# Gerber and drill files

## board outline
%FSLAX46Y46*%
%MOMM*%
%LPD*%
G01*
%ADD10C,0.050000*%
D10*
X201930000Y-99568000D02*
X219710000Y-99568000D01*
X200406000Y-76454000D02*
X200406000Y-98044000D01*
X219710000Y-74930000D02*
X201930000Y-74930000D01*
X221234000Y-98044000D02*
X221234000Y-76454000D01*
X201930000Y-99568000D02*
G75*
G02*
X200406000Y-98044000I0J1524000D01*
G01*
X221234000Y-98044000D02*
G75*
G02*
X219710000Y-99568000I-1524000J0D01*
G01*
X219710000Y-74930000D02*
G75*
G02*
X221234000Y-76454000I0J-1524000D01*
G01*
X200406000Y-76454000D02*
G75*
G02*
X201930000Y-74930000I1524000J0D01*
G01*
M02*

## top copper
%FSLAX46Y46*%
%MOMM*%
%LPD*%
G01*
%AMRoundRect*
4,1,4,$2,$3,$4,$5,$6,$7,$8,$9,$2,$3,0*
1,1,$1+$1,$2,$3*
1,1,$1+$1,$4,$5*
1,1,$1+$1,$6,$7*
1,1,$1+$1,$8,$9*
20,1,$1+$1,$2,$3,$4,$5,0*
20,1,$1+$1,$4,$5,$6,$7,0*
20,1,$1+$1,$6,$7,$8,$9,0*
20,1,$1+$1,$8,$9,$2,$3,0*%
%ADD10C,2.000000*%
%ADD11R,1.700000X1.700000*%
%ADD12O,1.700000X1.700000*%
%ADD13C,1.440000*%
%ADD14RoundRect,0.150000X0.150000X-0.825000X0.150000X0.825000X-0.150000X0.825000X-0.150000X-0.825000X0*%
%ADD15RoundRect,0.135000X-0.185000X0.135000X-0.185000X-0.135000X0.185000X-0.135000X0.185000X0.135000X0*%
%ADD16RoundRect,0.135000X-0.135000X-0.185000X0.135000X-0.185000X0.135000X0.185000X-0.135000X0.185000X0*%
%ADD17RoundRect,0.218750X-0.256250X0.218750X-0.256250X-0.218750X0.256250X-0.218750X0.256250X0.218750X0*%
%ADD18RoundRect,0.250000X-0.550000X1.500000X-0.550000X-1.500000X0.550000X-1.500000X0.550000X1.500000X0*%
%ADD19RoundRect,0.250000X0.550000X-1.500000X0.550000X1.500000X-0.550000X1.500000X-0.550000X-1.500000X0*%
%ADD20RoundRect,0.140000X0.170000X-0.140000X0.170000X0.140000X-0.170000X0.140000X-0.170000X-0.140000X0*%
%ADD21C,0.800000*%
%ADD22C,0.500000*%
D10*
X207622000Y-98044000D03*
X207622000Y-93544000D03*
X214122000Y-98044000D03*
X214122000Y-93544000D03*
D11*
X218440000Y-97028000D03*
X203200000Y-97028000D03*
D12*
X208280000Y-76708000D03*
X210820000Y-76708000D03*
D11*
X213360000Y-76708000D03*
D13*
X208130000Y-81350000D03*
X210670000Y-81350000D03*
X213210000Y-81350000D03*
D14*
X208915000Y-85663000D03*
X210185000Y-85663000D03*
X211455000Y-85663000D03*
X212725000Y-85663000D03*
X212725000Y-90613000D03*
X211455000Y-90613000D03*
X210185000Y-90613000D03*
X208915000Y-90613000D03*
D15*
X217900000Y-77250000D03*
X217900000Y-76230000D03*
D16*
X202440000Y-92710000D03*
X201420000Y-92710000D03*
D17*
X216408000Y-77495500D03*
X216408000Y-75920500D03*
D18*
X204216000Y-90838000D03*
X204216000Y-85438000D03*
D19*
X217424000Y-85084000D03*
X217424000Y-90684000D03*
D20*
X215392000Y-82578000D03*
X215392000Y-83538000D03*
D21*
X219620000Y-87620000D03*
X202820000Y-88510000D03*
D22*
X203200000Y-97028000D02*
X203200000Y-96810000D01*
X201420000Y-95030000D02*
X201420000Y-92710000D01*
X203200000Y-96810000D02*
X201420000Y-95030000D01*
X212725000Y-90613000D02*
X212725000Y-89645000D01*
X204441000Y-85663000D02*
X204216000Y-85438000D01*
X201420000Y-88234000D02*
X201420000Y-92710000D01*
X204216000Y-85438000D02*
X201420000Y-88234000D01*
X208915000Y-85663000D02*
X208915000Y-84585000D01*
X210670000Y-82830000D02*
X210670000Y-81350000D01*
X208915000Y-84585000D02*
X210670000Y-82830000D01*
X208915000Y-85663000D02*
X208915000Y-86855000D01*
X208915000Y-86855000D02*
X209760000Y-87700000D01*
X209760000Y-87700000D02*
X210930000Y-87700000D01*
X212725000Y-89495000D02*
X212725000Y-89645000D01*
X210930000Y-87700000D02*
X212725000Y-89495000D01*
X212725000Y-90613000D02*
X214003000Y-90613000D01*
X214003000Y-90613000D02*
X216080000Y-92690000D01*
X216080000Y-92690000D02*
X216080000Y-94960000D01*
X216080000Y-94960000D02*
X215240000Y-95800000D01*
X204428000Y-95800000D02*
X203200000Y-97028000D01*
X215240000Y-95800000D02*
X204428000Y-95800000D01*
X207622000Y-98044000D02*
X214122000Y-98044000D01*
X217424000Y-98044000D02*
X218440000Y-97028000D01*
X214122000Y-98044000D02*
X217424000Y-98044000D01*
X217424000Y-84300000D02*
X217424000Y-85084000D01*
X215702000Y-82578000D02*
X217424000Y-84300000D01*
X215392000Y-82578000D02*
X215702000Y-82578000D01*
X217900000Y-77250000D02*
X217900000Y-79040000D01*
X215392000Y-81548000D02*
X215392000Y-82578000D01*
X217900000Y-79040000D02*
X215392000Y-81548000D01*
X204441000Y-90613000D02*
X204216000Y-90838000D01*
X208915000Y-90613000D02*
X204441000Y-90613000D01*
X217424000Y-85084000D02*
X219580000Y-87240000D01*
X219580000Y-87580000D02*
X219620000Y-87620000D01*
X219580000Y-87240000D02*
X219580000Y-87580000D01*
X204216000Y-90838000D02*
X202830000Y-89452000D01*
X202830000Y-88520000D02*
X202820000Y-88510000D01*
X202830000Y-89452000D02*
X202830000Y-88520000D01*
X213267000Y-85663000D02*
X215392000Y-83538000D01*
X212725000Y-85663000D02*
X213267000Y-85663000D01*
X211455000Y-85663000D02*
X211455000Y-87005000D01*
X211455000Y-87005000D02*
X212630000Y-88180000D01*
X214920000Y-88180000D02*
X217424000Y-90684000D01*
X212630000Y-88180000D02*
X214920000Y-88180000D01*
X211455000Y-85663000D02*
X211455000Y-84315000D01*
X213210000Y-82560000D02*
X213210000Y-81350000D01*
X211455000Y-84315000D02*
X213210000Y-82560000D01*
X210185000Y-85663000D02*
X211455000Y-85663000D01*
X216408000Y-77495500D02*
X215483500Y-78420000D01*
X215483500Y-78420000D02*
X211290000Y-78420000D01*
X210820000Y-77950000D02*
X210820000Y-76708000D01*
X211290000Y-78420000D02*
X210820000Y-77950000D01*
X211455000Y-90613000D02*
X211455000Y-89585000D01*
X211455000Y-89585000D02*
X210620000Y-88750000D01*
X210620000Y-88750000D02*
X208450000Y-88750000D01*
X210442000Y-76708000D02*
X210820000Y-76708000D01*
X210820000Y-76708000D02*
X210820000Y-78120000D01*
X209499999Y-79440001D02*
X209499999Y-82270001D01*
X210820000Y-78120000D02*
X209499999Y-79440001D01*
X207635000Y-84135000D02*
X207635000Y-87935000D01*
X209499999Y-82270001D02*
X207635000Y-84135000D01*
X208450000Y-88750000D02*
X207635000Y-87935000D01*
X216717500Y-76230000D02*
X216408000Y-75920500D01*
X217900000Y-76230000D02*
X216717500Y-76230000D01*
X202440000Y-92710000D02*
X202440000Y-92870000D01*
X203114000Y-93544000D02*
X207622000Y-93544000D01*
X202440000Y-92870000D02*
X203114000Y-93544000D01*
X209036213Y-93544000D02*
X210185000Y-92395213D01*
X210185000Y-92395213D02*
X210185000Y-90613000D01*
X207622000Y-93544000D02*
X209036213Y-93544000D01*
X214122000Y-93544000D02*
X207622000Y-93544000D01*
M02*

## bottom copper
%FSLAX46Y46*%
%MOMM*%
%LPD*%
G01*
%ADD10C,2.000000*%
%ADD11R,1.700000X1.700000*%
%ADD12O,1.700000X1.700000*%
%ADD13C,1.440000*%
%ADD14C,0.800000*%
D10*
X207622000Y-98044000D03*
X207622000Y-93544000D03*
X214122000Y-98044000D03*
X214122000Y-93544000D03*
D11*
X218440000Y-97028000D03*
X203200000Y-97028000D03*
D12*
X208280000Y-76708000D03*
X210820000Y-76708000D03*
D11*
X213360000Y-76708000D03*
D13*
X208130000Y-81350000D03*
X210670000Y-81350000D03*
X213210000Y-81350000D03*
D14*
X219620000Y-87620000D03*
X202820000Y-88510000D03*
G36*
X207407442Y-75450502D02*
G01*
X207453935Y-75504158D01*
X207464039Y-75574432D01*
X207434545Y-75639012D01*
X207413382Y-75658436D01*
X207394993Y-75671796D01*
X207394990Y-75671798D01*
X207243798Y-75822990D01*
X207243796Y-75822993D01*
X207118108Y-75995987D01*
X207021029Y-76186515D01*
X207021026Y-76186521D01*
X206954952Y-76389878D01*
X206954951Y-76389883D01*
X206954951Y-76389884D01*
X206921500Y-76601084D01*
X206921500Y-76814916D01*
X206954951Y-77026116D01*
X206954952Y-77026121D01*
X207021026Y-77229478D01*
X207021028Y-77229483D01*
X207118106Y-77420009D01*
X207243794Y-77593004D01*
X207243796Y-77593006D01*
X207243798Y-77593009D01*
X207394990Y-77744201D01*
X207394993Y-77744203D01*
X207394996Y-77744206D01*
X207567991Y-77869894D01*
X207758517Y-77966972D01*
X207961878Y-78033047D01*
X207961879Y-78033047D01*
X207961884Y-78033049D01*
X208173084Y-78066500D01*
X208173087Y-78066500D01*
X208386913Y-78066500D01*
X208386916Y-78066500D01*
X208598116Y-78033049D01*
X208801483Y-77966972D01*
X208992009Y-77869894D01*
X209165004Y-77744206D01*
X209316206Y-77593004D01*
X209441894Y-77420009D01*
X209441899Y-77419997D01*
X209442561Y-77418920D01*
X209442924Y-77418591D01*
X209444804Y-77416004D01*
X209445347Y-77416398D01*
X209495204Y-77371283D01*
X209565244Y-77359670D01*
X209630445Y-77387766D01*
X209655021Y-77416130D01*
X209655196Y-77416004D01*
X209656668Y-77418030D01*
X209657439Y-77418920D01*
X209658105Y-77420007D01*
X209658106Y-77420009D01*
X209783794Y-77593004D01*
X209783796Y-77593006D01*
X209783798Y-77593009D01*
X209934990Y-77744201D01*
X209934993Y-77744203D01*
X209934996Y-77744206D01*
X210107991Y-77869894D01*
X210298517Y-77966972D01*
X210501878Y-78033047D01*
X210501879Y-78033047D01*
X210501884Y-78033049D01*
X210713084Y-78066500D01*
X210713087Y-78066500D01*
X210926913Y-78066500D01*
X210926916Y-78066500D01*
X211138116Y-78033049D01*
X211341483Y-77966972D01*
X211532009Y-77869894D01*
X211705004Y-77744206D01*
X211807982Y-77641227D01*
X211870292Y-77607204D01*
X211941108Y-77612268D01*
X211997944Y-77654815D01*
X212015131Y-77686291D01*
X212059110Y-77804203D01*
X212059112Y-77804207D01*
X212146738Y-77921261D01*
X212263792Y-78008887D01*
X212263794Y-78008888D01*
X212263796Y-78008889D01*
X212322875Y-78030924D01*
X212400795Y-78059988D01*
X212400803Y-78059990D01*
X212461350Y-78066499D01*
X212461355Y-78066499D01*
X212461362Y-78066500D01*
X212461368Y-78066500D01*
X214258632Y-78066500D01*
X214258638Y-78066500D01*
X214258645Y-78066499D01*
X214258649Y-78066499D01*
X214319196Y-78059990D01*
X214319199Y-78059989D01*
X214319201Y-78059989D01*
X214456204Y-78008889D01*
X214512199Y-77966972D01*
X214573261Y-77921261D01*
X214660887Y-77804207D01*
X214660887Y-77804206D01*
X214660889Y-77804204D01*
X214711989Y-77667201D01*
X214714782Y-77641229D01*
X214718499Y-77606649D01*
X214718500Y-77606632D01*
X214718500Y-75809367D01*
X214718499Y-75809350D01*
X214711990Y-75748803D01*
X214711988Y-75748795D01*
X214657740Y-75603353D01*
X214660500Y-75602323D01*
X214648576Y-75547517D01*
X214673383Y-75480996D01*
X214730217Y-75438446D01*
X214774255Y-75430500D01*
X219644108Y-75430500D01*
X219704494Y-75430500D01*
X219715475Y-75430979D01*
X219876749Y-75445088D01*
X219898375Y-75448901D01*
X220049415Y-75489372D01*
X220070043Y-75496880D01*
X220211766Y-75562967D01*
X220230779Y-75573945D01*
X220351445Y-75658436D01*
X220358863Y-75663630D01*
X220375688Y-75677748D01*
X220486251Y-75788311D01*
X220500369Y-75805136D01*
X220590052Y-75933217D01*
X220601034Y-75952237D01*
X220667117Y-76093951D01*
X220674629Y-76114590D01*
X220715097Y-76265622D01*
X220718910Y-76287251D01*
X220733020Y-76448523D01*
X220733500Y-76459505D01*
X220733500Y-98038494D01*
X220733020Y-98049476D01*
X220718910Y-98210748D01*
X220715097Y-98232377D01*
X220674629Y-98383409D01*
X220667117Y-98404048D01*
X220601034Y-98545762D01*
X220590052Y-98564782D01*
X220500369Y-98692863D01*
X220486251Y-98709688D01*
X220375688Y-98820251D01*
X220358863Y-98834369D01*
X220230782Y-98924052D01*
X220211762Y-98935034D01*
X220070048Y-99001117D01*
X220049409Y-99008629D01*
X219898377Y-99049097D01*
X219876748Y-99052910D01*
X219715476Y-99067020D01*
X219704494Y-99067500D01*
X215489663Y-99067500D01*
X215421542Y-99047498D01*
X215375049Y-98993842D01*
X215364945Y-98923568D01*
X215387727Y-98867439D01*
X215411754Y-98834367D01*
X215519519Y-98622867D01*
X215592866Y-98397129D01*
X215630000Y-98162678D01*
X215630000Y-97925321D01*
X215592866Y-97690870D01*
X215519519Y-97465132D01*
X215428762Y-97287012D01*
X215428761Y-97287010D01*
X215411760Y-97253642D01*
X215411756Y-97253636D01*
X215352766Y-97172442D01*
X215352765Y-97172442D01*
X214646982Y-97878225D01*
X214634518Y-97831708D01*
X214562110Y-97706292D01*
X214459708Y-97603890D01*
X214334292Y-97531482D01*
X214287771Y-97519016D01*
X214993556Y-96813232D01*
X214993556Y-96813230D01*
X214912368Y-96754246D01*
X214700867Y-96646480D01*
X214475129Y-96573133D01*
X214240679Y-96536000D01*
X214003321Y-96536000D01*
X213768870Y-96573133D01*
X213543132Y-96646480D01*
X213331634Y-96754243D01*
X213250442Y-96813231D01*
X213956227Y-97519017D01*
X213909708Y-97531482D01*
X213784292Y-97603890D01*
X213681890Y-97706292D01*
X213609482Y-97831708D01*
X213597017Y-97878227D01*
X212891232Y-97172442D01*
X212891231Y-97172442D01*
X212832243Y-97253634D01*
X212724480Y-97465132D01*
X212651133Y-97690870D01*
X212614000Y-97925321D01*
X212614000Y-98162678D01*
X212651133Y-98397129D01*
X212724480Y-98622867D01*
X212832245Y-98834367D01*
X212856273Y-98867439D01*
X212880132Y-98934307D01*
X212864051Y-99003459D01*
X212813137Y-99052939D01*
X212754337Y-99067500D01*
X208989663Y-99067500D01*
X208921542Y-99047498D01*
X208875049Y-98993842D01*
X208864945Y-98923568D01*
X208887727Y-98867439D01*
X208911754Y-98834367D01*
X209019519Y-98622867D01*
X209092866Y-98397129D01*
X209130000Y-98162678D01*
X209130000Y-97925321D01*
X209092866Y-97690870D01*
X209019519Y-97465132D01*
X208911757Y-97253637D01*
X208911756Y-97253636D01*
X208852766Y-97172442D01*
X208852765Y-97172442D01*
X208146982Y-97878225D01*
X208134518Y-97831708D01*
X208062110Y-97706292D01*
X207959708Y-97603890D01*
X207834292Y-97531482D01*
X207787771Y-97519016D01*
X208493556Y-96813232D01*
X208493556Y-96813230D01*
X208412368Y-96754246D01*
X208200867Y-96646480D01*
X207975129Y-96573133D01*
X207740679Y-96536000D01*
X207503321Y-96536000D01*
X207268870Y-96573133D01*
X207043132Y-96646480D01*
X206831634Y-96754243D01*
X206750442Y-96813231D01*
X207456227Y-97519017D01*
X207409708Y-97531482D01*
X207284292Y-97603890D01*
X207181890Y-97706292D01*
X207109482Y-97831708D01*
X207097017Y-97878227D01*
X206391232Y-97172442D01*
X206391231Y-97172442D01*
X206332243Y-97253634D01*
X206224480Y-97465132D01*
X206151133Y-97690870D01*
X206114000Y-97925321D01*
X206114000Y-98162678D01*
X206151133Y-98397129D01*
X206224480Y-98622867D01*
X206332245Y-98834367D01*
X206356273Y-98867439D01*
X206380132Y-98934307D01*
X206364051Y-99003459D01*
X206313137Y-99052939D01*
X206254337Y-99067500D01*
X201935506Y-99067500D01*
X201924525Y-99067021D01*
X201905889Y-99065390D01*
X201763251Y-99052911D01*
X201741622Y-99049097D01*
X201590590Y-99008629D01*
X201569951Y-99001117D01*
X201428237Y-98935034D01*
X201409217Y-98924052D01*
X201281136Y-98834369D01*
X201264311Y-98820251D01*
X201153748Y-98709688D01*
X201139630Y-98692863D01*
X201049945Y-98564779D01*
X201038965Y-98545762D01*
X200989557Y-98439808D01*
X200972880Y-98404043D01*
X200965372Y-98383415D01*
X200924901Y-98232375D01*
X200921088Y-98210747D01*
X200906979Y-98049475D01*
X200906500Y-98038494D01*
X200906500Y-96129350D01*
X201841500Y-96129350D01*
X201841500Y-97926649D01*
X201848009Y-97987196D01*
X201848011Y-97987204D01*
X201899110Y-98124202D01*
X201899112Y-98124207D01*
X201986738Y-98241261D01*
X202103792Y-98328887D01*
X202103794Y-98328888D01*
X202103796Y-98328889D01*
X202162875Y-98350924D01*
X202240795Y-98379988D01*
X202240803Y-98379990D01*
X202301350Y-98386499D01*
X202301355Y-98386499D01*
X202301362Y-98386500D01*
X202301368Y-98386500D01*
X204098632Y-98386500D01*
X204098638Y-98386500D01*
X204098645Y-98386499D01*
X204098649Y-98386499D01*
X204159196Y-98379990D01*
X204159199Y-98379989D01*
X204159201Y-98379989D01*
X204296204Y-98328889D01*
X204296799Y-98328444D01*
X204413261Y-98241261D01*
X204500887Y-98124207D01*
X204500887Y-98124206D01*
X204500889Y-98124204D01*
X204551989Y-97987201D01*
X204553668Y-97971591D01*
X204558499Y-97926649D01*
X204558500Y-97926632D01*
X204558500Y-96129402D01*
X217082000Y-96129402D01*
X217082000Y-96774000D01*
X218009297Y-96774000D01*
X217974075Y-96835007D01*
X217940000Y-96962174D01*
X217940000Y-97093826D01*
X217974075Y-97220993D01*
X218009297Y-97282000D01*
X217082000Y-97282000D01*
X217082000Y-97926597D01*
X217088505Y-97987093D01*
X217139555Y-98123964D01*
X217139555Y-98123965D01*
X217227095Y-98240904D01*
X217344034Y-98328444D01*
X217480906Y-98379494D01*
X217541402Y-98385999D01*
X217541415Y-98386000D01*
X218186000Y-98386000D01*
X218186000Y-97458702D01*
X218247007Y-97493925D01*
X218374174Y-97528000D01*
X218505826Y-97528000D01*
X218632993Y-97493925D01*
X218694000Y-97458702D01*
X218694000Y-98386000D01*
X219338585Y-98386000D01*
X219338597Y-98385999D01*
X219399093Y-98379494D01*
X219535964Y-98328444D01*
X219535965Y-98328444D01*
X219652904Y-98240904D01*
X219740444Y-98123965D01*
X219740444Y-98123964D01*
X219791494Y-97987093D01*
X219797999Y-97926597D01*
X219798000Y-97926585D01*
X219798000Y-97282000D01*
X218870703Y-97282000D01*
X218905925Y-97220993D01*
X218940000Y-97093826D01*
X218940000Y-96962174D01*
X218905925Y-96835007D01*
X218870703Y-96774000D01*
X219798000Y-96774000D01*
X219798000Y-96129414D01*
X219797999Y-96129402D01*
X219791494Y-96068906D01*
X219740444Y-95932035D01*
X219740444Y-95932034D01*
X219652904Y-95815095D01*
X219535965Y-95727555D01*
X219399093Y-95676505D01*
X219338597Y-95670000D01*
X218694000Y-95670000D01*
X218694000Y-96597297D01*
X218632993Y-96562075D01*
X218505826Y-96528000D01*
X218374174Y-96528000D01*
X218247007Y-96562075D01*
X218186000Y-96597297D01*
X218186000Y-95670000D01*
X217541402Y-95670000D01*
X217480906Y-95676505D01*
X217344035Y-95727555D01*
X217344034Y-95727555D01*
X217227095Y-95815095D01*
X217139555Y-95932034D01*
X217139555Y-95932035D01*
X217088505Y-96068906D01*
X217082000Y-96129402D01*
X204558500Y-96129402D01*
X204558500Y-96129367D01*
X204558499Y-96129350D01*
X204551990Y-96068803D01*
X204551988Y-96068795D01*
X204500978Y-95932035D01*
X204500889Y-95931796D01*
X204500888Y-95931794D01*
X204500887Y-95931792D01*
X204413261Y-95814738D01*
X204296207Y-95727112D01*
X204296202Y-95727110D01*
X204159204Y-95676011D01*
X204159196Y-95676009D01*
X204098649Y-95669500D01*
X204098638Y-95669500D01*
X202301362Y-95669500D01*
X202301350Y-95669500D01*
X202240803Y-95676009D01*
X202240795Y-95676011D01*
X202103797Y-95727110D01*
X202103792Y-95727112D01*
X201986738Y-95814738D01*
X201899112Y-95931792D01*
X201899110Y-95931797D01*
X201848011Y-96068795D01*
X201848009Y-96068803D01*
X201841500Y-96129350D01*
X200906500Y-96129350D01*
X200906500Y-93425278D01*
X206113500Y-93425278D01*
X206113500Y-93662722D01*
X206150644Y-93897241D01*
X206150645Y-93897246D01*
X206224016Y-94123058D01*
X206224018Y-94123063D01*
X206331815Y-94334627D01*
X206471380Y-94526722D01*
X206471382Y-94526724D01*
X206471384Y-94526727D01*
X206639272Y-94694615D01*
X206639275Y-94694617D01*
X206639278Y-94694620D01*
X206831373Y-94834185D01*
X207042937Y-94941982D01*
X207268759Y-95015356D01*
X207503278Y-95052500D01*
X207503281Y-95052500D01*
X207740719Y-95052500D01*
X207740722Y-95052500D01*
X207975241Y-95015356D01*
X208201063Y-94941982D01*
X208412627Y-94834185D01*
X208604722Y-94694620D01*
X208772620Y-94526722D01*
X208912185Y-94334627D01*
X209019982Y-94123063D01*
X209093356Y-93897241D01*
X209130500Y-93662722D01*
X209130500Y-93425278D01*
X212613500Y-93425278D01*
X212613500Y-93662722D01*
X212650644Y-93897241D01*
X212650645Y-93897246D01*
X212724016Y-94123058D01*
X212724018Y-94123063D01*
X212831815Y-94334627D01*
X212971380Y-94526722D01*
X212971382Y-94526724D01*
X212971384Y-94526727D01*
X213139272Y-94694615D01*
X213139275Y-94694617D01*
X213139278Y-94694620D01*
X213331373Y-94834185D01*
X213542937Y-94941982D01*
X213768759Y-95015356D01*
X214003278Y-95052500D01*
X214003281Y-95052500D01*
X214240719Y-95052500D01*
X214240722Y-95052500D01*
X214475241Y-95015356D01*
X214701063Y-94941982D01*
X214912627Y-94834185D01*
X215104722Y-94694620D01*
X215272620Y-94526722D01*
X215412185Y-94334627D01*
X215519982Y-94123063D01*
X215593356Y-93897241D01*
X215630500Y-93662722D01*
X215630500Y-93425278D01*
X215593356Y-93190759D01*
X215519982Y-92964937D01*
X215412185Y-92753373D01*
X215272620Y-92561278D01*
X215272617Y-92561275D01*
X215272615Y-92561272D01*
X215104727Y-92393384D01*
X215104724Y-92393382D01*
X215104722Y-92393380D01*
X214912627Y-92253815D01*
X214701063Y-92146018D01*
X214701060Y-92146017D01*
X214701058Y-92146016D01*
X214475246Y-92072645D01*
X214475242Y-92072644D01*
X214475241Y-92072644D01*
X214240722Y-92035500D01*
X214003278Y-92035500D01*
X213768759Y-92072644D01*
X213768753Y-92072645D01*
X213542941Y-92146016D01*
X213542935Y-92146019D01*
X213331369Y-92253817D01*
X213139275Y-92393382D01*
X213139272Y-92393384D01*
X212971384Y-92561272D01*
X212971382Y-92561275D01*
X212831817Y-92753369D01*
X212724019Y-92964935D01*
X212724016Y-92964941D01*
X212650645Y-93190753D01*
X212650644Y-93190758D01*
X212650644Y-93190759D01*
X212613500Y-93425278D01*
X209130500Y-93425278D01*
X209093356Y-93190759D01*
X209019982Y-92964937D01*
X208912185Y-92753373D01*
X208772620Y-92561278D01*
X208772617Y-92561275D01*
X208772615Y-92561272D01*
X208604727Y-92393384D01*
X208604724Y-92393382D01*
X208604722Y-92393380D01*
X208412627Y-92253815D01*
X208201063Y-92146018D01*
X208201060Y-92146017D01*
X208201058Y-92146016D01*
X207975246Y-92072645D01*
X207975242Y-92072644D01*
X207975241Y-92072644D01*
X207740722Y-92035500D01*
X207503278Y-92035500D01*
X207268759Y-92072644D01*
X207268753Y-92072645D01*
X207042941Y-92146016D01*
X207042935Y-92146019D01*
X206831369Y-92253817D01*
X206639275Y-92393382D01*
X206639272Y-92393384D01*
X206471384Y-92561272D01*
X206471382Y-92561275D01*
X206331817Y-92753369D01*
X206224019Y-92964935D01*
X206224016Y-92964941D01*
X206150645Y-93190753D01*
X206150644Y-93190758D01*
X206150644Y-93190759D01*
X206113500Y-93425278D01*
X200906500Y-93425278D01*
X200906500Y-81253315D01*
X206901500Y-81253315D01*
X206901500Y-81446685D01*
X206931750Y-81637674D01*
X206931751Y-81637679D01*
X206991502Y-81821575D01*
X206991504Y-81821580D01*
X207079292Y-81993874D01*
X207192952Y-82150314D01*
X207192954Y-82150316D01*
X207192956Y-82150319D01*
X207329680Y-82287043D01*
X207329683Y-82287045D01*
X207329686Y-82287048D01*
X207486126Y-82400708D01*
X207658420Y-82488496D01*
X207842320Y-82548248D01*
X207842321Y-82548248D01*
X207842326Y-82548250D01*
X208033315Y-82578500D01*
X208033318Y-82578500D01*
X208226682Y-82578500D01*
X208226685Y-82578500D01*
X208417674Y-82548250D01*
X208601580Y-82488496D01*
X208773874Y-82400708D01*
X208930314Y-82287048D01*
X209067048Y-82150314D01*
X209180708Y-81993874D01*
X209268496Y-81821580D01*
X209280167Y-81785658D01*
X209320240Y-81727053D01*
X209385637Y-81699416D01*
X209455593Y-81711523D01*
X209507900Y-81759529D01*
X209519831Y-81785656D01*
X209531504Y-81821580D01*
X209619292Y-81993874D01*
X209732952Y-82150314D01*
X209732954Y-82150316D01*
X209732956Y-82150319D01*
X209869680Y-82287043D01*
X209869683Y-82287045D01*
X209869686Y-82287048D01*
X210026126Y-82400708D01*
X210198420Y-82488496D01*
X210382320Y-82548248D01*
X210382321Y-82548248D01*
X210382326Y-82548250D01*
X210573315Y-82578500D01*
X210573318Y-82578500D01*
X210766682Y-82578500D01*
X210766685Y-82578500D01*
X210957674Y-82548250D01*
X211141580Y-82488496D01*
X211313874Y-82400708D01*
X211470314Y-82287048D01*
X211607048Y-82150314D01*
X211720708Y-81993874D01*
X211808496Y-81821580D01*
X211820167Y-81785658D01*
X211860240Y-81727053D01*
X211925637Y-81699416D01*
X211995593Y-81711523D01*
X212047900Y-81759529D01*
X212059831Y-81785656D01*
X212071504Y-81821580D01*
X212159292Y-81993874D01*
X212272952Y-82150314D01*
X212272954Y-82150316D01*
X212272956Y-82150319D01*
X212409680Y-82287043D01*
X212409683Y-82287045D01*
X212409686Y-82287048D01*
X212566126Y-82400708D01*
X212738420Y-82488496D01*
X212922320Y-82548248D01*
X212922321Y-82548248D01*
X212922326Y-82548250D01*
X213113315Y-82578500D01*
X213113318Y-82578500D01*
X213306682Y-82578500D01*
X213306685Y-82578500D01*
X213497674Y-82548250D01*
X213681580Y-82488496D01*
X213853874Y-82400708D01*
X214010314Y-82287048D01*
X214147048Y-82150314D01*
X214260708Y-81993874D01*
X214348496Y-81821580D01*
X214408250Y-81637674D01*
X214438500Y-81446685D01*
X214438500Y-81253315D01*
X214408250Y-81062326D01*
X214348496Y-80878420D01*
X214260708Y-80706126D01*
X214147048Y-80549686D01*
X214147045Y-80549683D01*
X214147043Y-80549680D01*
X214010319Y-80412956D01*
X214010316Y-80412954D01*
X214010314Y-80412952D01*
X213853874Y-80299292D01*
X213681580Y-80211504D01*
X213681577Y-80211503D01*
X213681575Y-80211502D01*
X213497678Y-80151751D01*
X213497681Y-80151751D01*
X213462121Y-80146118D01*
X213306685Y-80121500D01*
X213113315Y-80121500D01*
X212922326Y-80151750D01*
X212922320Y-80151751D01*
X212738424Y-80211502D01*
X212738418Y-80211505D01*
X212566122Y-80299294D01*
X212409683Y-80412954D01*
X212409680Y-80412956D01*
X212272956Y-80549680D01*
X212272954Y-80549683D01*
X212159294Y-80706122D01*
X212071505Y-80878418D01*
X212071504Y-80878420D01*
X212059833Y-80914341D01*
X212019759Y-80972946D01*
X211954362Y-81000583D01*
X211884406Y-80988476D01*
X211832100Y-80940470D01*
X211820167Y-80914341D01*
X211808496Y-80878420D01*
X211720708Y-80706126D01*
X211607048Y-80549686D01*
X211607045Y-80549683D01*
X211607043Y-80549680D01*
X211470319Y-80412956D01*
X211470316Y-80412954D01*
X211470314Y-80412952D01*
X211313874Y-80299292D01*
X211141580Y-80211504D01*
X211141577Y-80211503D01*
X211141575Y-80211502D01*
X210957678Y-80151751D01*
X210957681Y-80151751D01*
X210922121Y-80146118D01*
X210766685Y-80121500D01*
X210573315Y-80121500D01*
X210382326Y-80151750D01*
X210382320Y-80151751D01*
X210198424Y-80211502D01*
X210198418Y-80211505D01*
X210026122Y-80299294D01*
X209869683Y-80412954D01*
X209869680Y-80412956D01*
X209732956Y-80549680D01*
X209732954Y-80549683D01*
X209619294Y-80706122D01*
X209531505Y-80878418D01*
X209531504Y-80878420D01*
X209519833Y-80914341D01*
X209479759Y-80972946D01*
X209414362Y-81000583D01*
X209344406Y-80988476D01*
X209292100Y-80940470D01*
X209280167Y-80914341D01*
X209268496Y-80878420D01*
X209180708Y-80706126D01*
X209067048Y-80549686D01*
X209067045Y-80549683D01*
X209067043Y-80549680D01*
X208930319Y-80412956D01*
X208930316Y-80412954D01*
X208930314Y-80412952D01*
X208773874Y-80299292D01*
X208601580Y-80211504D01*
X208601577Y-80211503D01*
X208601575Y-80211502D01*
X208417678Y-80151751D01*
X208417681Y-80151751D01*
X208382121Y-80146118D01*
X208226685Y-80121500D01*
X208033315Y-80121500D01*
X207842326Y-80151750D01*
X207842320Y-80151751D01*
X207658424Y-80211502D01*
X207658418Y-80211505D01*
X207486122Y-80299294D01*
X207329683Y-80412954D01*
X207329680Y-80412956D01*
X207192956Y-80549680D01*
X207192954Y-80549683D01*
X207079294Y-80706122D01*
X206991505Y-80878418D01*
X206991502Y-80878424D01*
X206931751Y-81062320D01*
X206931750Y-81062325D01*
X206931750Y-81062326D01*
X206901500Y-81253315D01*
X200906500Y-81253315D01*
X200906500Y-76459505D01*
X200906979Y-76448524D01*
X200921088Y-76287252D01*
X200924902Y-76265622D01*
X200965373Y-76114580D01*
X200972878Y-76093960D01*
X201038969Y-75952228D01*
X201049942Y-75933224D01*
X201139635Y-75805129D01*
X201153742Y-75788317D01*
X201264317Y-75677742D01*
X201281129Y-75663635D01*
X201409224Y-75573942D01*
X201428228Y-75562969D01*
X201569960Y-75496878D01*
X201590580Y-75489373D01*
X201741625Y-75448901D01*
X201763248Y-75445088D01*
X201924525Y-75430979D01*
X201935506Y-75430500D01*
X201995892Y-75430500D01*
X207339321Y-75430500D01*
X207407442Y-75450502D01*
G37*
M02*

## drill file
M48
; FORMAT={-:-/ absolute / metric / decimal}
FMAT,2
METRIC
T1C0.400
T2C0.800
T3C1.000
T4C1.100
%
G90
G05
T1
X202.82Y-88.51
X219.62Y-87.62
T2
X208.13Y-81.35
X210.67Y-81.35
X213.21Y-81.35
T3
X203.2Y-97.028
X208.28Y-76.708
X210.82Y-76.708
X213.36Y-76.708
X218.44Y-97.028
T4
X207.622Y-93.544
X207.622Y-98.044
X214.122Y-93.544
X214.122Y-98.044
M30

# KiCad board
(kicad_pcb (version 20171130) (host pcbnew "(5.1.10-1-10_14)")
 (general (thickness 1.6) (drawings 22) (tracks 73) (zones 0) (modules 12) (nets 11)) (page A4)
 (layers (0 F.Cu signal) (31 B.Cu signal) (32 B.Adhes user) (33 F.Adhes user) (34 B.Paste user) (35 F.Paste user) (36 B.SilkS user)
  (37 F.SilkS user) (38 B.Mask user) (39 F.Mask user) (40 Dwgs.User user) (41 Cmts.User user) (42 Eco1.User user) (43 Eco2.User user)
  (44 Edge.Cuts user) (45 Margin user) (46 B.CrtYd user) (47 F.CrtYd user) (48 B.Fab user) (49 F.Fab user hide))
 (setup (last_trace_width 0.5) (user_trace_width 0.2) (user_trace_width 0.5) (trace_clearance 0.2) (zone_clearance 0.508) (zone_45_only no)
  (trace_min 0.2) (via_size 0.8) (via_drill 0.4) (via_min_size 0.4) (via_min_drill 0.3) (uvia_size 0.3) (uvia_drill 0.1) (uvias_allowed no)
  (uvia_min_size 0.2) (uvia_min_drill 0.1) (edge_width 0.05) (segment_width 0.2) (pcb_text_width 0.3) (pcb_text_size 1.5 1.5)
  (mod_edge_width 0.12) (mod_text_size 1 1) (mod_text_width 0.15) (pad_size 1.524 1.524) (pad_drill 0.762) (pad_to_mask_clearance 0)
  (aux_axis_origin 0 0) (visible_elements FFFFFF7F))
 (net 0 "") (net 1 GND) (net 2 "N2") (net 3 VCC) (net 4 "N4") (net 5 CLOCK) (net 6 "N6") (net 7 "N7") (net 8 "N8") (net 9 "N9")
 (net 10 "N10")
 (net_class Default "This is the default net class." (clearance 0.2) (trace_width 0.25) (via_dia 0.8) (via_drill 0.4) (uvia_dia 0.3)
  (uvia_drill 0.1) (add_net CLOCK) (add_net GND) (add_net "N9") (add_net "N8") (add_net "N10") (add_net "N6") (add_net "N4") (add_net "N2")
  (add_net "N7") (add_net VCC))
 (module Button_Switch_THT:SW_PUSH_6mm (layer F.Cu) (at 214.122 98.044 180)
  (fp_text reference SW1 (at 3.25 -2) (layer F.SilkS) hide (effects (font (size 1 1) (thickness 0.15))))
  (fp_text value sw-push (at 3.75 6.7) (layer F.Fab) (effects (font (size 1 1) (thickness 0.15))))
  (pad 1 thru_hole circle (at 6.5 0 270) (size 2 2) (drill 1.1) (layers *.Cu *.Mask) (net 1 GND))
  (pad 2 thru_hole circle (at 6.5 4.5 270) (size 2 2) (drill 1.1) (layers *.Cu *.Mask) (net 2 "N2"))
  (pad 1 thru_hole circle (at 0 0 270) (size 2 2) (drill 1.1) (layers *.Cu *.Mask) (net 1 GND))
  (pad 2 thru_hole circle (at 0 4.5 270) (size 2 2) (drill 1.1) (layers *.Cu *.Mask) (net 2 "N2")))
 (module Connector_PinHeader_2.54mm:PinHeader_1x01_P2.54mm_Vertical (layer B.Cu) (at 218.44 97.028)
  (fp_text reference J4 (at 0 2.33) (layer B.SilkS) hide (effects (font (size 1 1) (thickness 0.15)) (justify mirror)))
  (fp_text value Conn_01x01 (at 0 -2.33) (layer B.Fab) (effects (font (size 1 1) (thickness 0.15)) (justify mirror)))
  (pad 1 thru_hole rect (at 0 0) (size 1.7 1.7) (drill 1) (layers *.Cu *.Mask) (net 1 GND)))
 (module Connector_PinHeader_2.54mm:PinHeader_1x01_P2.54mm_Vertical (layer B.Cu) (at 203.2 97.028)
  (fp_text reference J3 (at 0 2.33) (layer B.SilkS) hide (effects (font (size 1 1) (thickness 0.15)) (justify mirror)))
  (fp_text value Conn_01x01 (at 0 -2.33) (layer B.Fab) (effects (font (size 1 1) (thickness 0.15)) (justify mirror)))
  (pad 1 thru_hole rect (at 0 0) (size 1.7 1.7) (drill 1) (layers *.Cu *.Mask) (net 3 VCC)))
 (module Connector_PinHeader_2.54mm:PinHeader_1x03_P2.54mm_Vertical (layer B.Cu) (at 213.36 76.708 90)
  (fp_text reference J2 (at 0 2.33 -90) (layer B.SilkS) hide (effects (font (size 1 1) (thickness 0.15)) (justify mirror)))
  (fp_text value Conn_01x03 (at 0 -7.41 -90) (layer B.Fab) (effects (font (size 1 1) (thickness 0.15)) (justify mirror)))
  (pad 3 thru_hole oval (at 0 -5.08 90) (size 1.7 1.7) (drill 1) (layers *.Cu *.Mask) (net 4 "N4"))
  (pad 2 thru_hole oval (at 0 -2.54 90) (size 1.7 1.7) (drill 1) (layers *.Cu *.Mask) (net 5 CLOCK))
  (pad 1 thru_hole rect (at 0 0 90) (size 1.7 1.7) (drill 1) (layers *.Cu *.Mask) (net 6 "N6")))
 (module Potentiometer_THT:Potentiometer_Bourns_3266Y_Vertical (layer F.Cu) (at 213.21 81.35)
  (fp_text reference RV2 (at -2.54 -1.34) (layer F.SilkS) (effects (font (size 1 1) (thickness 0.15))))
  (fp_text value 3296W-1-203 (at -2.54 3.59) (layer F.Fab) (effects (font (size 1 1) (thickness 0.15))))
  (pad 3 thru_hole circle (at -5.08 0) (size 1.44 1.44) (drill 0.8) (layers *.Cu *.Mask) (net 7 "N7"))
  (pad 2 thru_hole circle (at -2.54 0) (size 1.44 1.44) (drill 0.8) (layers *.Cu *.Mask) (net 3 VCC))
  (pad 1 thru_hole circle (at 0 0) (size 1.44 1.44) (drill 0.8) (layers *.Cu *.Mask) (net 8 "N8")))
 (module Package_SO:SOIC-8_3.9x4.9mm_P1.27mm (layer F.Cu) (at 210.82 88.138 90)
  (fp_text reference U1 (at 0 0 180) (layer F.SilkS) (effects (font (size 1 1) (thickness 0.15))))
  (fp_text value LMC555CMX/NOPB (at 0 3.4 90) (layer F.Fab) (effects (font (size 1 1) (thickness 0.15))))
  (pad 8 smd roundrect (at 2.475 -1.905 90) (size 1.95 0.6) (layers F.Cu F.Paste F.Mask) (roundrect_rratio 0.25) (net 3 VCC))
  (pad 7 smd roundrect (at 2.475 -0.635 90) (size 1.95 0.6) (layers F.Cu F.Paste F.Mask) (roundrect_rratio 0.25) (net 8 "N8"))
  (pad 6 smd roundrect (at 2.475 0.635 90) (size 1.95 0.6) (layers F.Cu F.Paste F.Mask) (roundrect_rratio 0.25) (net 8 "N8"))
  (pad 5 smd roundrect (at 2.475 1.905 90) (size 1.95 0.6) (layers F.Cu F.Paste F.Mask) (roundrect_rratio 0.25) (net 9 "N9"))
  (pad 4 smd roundrect (at -2.475 1.905 90) (size 1.95 0.6) (layers F.Cu F.Paste F.Mask) (roundrect_rratio 0.25) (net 3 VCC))
  (pad 3 smd roundrect (at -2.475 0.635 90) (size 1.95 0.6) (layers F.Cu F.Paste F.Mask) (roundrect_rratio 0.25) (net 5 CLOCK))
  (pad 2 smd roundrect (at -2.475 -0.635 90) (size 1.95 0.6) (layers F.Cu F.Paste F.Mask) (roundrect_rratio 0.25) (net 2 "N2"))
  (pad 1 smd roundrect (at -2.475 -1.905 90) (size 1.95 0.6) (layers F.Cu F.Paste F.Mask) (roundrect_rratio 0.25) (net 1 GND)))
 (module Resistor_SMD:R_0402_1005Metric (layer F.Cu) (at 217.9 76.74 270)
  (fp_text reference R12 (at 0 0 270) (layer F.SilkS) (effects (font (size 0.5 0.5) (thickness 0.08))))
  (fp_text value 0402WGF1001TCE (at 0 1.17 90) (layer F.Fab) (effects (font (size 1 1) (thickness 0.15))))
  (pad 2 smd roundrect (at 0.51 0 270) (size 0.54 0.64) (layers F.Cu F.Paste F.Mask) (roundrect_rratio 0.25) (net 1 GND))
  (pad 1 smd roundrect (at -0.51 0 270) (size 0.54 0.64) (layers F.Cu F.Paste F.Mask) (roundrect_rratio 0.25) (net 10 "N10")))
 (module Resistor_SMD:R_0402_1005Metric (layer F.Cu) (at 201.93 92.71)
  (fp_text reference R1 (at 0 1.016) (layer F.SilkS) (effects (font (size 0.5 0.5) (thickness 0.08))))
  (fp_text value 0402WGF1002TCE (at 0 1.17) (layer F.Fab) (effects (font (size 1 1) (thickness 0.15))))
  (pad 2 smd roundrect (at 0.51 0) (size 0.54 0.64) (layers F.Cu F.Paste F.Mask) (roundrect_rratio 0.25) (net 2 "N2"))
  (pad 1 smd roundrect (at -0.51 0) (size 0.54 0.64) (layers F.Cu F.Paste F.Mask) (roundrect_rratio 0.25) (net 3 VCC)))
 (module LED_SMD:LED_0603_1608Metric (layer F.Cu) (at 216.408 76.708 270)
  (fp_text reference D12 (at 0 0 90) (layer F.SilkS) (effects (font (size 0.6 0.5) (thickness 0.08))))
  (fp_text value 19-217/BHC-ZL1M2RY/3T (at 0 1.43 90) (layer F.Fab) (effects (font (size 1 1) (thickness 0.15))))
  (pad 2 smd roundrect (at 0.7875 0 270) (size 0.875 0.95) (layers F.Cu F.Paste F.Mask) (roundrect_rratio 0.25) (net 5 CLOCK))
  (pad 1 smd roundrect (at -0.7875 0 270) (size 0.875 0.95) (layers F.Cu F.Paste F.Mask) (roundrect_rratio 0.25) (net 10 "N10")))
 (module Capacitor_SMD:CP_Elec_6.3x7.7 (layer F.Cu) (at 204.216 88.138 270)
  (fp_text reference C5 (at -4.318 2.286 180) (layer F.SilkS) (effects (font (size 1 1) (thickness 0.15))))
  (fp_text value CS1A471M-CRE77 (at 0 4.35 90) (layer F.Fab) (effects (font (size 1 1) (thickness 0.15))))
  (pad 2 smd roundrect (at 2.7 0 270) (size 3.5 1.6) (layers F.Cu F.Paste F.Mask) (roundrect_rratio 0.15625) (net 1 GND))
  (pad 1 smd roundrect (at -2.7 0 270) (size 3.5 1.6) (layers F.Cu F.Paste F.Mask) (roundrect_rratio 0.15625) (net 3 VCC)))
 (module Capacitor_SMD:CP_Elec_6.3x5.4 (layer F.Cu) (at 217.424 87.884 90)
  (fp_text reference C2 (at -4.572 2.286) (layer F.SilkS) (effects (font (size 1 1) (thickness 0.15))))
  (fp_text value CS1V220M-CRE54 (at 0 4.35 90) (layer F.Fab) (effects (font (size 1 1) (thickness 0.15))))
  (pad 2 smd roundrect (at 2.8 0 90) (size 3.5 1.6) (layers F.Cu F.Paste F.Mask) (roundrect_rratio 0.15625) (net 1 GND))
  (pad 1 smd roundrect (at -2.8 0 90) (size 3.5 1.6) (layers F.Cu F.Paste F.Mask) (roundrect_rratio 0.15625) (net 8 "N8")))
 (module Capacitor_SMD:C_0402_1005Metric (layer F.Cu) (at 215.392 83.058 90)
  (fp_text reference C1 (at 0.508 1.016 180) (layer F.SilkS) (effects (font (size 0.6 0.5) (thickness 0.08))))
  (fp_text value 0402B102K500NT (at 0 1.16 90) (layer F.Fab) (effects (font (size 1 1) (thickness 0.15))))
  (pad 2 smd roundrect (at 0.48 0 90) (size 0.56 0.62) (layers F.Cu F.Paste F.Mask) (roundrect_rratio 0.25) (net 1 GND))
  (pad 1 smd roundrect (at -0.48 0 90) (size 0.56 0.62) (layers F.Cu F.Paste F.Mask) (roundrect_rratio 0.25) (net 9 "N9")))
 (gr_line (start 201.93 99.568) (end 219.71 99.568) (layer Edge.Cuts) (width 0.05))
 (gr_line (start 200.406 76.454) (end 200.406 98.044) (layer Edge.Cuts) (width 0.05))
 (gr_line (start 219.71 74.93) (end 201.93 74.93) (layer Edge.Cuts) (width 0.05))
 (gr_line (start 221.234 98.044) (end 221.234 76.454) (layer Edge.Cuts) (width 0.05))
 (gr_arc (start 201.93 98.044) (end 200.406 98.044) (angle -90) (layer Edge.Cuts) (width 0.05))
 (gr_arc (start 219.71 98.044) (end 219.71 99.568) (angle -90) (layer Edge.Cuts) (width 0.05))
 (gr_arc (start 219.71 76.454) (end 221.234 76.454) (angle -90) (layer Edge.Cuts) (width 0.05))
 (gr_arc (start 201.93 76.454) (end 201.93 74.93) (angle -90) (layer Edge.Cuts) (width 0.05))
 (segment (start 203.2 97.028) (end 203.2 96.81) (width 0.5) (layer F.Cu) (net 3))
 (segment (start 201.42 95.03) (end 201.42 92.71) (width 0.5) (layer F.Cu) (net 3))
 (segment (start 203.2 96.81) (end 201.42 95.03) (width 0.5) (layer F.Cu) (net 3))
 (segment (start 212.725 90.613) (end 212.725 89.645) (width 0.5) (layer F.Cu) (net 3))
 (segment (start 204.441 85.663) (end 204.216 85.438) (width 0.5) (layer F.Cu) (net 3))
 (segment (start 201.42 88.234) (end 201.42 92.71) (width 0.5) (layer F.Cu) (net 3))
 (segment (start 204.216 85.438) (end 201.42 88.234) (width 0.5) (layer F.Cu) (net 3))
 (segment (start 208.915 85.663) (end 208.915 84.585) (width 0.5) (layer F.Cu) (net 3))
 (segment (start 210.67 82.83) (end 210.67 81.35) (width 0.5) (layer F.Cu) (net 3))
 (segment (start 208.915 84.585) (end 210.67 82.83) (width 0.5) (layer F.Cu) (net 3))
 (segment (start 208.915 85.663) (end 208.915 86.855) (width 0.5) (layer F.Cu) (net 3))
 (segment (start 208.915 86.855) (end 209.76 87.7) (width 0.5) (layer F.Cu) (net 3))
 (segment (start 209.76 87.7) (end 210.93 87.7) (width 0.5) (layer F.Cu) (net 3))
 (segment (start 212.725 89.495) (end 212.725 89.645) (width 0.5) (layer F.Cu) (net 3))
 (segment (start 210.93 87.7) (end 212.725 89.495) (width 0.5) (layer F.Cu) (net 3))
 (segment (start 212.725 90.613) (end 214.003 90.613) (width 0.5) (layer F.Cu) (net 3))
 (segment (start 214.003 90.613) (end 216.08 92.69) (width 0.5) (layer F.Cu) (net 3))
 (segment (start 216.08 92.69) (end 216.08 94.96) (width 0.5) (layer F.Cu) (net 3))
 (segment (start 216.08 94.96) (end 215.24 95.8) (width 0.5) (layer F.Cu) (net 3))
 (segment (start 204.428 95.8) (end 203.2 97.028) (width 0.5) (layer F.Cu) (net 3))
 (segment (start 215.24 95.8) (end 204.428 95.8) (width 0.5) (layer F.Cu) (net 3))
 (segment (start 207.622 98.044) (end 214.122 98.044) (width 0.5) (layer F.Cu) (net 1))
 (segment (start 217.424 98.044) (end 218.44 97.028) (width 0.5) (layer F.Cu) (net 1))
 (segment (start 214.122 98.044) (end 217.424 98.044) (width 0.5) (layer F.Cu) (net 1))
 (segment (start 217.424 84.3) (end 217.424 85.084) (width 0.5) (layer F.Cu) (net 1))
 (segment (start 215.702 82.578) (end 217.424 84.3) (width 0.5) (layer F.Cu) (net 1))
 (segment (start 215.392 82.578) (end 215.702 82.578) (width 0.5) (layer F.Cu) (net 1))
 (segment (start 217.9 77.25) (end 217.9 79.04) (width 0.5) (layer F.Cu) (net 1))
 (segment (start 215.392 81.548) (end 215.392 82.578) (width 0.5) (layer F.Cu) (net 1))
 (segment (start 217.9 79.04) (end 215.392 81.548) (width 0.5) (layer F.Cu) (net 1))
 (segment (start 204.441 90.613) (end 204.216 90.838) (width 0.5) (layer F.Cu) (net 1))
 (segment (start 208.915 90.613) (end 204.441 90.613) (width 0.5) (layer F.Cu) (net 1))
 (segment (start 217.424 85.084) (end 219.58 87.24) (width 0.5) (layer F.Cu) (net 1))
 (via (at 219.62 87.62) (size 0.8) (drill 0.4) (layers F.Cu B.Cu) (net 1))
 (segment (start 219.58 87.58) (end 219.62 87.62) (width 0.5) (layer F.Cu) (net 1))
 (segment (start 219.58 87.24) (end 219.58 87.58) (width 0.5) (layer F.Cu) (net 1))
 (segment (start 204.216 90.838) (end 202.83 89.452) (width 0.5) (layer F.Cu) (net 1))
 (via (at 202.82 88.51) (size 0.8) (drill 0.4) (layers F.Cu B.Cu) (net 1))
 (segment (start 202.83 88.52) (end 202.82 88.51) (width 0.5) (layer F.Cu) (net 1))
 (segment (start 202.83 89.452) (end 202.83 88.52) (width 0.5) (layer F.Cu) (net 1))
 (segment (start 213.267 85.663) (end 215.392 83.538) (width 0.5) (layer F.Cu) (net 9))
 (segment (start 212.725 85.663) (end 213.267 85.663) (width 0.5) (layer F.Cu) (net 9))
 (segment (start 211.455 85.663) (end 211.455 87.005) (width 0.5) (layer F.Cu) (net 8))
 (segment (start 211.455 87.005) (end 212.63 88.18) (width 0.5) (layer F.Cu) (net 8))
 (segment (start 214.92 88.18) (end 217.424 90.684) (width 0.5) (layer F.Cu) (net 8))
 (segment (start 212.63 88.18) (end 214.92 88.18) (width 0.5) (layer F.Cu) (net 8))
 (segment (start 211.455 85.663) (end 211.455 84.315) (width 0.5) (layer F.Cu) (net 8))
 (segment (start 213.21 82.56) (end 213.21 81.35) (width 0.5) (layer F.Cu) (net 8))
 (segment (start 211.455 84.315) (end 213.21 82.56) (width 0.5) (layer F.Cu) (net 8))
 (segment (start 210.185 85.663) (end 211.455 85.663) (width 0.5) (layer F.Cu) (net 8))
 (segment (start 216.408 77.4955) (end 215.4835 78.42) (width 0.5) (layer F.Cu) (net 5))
 (segment (start 215.4835 78.42) (end 211.29 78.42) (width 0.5) (layer F.Cu) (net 5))
 (segment (start 210.82 77.95) (end 210.82 76.708) (width 0.5) (layer F.Cu) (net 5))
 (segment (start 211.29 78.42) (end 210.82 77.95) (width 0.5) (layer F.Cu) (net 5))
 (segment (start 211.455 90.613) (end 211.455 89.585) (width 0.5) (layer F.Cu) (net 5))
 (segment (start 211.455 89.585) (end 210.62 88.75) (width 0.5) (layer F.Cu) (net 5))
 (segment (start 210.62 88.75) (end 208.45 88.75) (width 0.5) (layer F.Cu) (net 5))
 (segment (start 210.442 76.708) (end 210.82 76.708) (width 0.5) (layer F.Cu) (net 5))
 (segment (start 210.82 76.708) (end 210.82 78.12) (width 0.5) (layer F.Cu) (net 5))
 (segment (start 209.499999 79.440001) (end 209.499999 82.270001) (width 0.5) (layer F.Cu) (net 5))
 (segment (start 210.82 78.12) (end 209.499999 79.440001) (width 0.5) (layer F.Cu) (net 5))
 (segment (start 207.635 84.135) (end 207.635 87.935) (width 0.5) (layer F.Cu) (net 5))
 (segment (start 209.499999 82.270001) (end 207.635 84.135) (width 0.5) (layer F.Cu) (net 5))
 (segment (start 208.45 88.75) (end 207.635 87.935) (width 0.5) (layer F.Cu) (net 5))
 (segment (start 216.7175 76.23) (end 216.408 75.9205) (width 0.5) (layer F.Cu) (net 10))
 (segment (start 217.9 76.23) (end 216.7175 76.23) (width 0.5) (layer F.Cu) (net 10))
 (segment (start 202.44 92.71) (end 202.44 92.87) (width 0.5) (layer F.Cu) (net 2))
 (segment (start 203.114 93.544) (end 207.622 93.544) (width 0.5) (layer F.Cu) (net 2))
 (segment (start 202.44 92.87) (end 203.114 93.544) (width 0.5) (layer F.Cu) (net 2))
 (segment (start 209.036213 93.544) (end 210.185 92.395213) (width 0.5) (layer F.Cu) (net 2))
 (segment (start 210.185 92.395213) (end 210.185 90.613) (width 0.5) (layer F.Cu) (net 2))
 (segment (start 207.622 93.544) (end 209.036213 93.544) (width 0.5) (layer F.Cu) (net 2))
 (segment (start 214.122 93.544) (end 207.622 93.544) (width 0.5) (layer F.Cu) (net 2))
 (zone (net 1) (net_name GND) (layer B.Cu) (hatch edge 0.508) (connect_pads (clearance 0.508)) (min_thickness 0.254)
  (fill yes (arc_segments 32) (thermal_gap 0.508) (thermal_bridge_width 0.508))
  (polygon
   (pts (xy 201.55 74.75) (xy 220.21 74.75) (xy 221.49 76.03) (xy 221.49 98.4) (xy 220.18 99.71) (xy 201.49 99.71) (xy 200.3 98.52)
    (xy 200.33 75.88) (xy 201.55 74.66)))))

